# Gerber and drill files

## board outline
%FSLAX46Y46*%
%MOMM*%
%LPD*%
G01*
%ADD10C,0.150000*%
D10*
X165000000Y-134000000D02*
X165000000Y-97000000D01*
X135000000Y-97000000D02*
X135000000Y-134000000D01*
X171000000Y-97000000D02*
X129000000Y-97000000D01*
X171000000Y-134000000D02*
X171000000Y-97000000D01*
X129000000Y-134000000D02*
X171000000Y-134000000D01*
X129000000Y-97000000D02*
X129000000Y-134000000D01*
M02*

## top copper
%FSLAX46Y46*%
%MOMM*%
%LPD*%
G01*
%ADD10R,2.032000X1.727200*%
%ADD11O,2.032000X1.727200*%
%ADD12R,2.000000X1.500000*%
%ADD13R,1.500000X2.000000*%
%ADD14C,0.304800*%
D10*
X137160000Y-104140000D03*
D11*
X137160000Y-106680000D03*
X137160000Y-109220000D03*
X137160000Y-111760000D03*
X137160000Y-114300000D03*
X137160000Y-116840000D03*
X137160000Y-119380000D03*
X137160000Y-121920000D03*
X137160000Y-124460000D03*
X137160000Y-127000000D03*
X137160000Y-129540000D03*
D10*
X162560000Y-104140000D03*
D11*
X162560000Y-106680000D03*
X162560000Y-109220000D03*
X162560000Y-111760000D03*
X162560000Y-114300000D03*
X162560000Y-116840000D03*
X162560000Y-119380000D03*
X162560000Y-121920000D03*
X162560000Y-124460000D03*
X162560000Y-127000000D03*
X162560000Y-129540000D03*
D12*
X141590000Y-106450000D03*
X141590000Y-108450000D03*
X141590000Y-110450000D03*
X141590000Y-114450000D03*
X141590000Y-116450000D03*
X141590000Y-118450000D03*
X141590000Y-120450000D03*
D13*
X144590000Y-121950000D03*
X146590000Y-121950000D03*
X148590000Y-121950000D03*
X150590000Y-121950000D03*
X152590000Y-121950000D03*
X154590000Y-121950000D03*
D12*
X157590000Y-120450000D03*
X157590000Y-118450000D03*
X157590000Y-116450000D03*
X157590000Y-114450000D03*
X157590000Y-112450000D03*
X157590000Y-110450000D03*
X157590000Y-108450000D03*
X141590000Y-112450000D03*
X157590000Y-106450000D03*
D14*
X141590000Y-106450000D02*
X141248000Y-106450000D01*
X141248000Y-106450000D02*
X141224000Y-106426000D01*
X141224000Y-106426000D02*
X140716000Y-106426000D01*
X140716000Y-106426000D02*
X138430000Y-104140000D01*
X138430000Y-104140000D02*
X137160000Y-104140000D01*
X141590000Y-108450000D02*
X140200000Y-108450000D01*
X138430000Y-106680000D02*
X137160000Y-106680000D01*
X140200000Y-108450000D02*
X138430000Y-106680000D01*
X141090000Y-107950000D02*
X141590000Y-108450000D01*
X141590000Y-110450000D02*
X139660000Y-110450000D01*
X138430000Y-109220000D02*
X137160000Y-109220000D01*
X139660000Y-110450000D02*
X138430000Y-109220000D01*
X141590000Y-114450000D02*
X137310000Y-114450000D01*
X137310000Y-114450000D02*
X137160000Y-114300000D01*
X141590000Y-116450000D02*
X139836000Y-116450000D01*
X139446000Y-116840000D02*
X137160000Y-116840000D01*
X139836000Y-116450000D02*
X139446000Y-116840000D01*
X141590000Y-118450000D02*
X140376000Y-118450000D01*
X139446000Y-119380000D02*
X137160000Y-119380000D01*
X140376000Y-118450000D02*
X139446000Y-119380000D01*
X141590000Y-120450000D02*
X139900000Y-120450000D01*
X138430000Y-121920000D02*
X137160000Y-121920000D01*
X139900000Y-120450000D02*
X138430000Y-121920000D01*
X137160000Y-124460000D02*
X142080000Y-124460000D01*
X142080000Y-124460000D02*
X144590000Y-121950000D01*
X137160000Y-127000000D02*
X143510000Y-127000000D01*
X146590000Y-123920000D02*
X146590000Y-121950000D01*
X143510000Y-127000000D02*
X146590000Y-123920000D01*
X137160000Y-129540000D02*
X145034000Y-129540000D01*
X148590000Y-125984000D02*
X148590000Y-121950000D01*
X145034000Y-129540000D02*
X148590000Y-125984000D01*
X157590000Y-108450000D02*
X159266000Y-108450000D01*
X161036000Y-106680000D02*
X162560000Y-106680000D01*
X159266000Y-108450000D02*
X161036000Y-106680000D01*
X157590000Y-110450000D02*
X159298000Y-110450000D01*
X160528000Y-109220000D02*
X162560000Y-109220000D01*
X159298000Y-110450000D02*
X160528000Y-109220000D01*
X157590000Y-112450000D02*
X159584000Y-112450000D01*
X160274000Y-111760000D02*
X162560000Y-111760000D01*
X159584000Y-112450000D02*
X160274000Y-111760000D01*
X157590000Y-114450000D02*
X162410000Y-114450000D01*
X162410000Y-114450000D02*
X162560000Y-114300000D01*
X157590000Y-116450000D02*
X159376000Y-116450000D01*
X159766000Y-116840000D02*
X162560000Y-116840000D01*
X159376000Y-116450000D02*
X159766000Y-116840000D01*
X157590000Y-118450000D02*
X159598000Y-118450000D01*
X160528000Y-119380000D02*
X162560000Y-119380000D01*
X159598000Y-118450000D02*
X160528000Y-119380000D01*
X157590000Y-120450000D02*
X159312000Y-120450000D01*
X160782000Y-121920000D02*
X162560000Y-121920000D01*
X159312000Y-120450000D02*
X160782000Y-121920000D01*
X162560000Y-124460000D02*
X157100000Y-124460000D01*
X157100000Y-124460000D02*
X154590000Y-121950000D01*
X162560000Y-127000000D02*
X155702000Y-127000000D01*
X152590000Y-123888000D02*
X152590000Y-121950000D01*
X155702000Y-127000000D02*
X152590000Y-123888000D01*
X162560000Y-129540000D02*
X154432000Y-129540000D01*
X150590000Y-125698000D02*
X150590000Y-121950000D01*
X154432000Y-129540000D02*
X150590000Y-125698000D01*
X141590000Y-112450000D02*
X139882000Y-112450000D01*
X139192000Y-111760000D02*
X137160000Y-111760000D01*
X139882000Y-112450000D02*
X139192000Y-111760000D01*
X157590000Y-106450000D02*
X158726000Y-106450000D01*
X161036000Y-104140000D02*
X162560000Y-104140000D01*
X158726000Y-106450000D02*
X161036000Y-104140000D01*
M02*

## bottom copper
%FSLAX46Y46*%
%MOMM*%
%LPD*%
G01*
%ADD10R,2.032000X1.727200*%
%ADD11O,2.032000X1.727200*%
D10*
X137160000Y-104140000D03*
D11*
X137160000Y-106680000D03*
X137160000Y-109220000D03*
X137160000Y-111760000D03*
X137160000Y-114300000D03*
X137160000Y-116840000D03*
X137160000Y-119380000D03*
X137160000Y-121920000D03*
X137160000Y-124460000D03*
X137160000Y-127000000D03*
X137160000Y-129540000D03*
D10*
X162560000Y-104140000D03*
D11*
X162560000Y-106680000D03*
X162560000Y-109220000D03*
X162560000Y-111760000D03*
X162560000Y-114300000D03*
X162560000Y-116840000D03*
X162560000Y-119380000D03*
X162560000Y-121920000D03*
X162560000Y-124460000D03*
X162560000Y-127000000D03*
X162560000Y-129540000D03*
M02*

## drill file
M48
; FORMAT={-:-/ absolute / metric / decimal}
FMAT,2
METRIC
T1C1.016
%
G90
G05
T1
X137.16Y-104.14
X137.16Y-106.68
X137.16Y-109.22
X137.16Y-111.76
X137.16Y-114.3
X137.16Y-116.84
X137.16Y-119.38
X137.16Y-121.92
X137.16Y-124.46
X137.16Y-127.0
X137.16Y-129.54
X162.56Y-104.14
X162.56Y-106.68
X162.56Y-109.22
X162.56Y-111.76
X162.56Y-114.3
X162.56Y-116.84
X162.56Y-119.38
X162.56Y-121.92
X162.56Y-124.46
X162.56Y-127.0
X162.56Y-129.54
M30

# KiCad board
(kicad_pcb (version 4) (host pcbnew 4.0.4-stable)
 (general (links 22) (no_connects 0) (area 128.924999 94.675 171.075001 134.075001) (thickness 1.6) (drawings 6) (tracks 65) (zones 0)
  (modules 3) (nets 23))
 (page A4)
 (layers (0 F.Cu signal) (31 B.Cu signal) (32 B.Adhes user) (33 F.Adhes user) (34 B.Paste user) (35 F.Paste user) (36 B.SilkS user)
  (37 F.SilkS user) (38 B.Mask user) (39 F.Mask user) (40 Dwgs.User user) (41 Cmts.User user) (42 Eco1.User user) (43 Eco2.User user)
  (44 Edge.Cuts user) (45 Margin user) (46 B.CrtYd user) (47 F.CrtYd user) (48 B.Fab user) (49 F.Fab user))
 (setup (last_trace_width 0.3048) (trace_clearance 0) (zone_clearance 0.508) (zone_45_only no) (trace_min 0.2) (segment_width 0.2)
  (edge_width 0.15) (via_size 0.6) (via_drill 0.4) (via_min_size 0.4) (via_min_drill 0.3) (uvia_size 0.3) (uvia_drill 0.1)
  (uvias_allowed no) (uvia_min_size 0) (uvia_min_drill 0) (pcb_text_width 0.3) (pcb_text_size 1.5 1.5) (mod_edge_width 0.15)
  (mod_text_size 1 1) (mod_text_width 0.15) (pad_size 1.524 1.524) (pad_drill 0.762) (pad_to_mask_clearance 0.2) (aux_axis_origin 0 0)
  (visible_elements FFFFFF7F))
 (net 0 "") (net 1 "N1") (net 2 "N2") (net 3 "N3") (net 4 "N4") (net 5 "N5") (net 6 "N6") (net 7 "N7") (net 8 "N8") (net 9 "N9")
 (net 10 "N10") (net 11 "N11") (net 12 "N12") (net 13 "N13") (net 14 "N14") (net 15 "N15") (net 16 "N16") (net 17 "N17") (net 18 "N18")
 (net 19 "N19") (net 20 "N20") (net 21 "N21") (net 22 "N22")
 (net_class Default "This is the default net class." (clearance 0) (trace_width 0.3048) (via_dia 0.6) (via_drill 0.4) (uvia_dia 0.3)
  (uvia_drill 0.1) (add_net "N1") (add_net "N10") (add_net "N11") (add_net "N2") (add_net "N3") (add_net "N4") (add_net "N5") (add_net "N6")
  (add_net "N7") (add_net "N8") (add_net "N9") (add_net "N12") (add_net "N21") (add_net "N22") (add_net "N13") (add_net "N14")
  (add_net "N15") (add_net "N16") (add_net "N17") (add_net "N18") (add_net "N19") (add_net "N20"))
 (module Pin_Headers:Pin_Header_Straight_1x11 (layer F.Cu) (at 137.16 104.14)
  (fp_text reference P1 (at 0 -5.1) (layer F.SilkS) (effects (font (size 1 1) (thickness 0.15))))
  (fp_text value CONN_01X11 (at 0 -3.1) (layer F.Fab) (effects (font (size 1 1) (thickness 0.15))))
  (pad 1 thru_hole rect (at 0 0) (size 2.032 1.7272) (drill 1.016) (layers *.Cu *.Mask F.SilkS) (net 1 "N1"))
  (pad 2 thru_hole oval (at 0 2.54) (size 2.032 1.7272) (drill 1.016) (layers *.Cu *.Mask F.SilkS) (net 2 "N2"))
  (pad 3 thru_hole oval (at 0 5.08) (size 2.032 1.7272) (drill 1.016) (layers *.Cu *.Mask F.SilkS) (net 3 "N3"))
  (pad 4 thru_hole oval (at 0 7.62) (size 2.032 1.7272) (drill 1.016) (layers *.Cu *.Mask F.SilkS) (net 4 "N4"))
  (pad 5 thru_hole oval (at 0 10.16) (size 2.032 1.7272) (drill 1.016) (layers *.Cu *.Mask F.SilkS) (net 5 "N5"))
  (pad 6 thru_hole oval (at 0 12.7) (size 2.032 1.7272) (drill 1.016) (layers *.Cu *.Mask F.SilkS) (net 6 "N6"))
  (pad 7 thru_hole oval (at 0 15.24) (size 2.032 1.7272) (drill 1.016) (layers *.Cu *.Mask F.SilkS) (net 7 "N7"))
  (pad 8 thru_hole oval (at 0 17.78) (size 2.032 1.7272) (drill 1.016) (layers *.Cu *.Mask F.SilkS) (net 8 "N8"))
  (pad 9 thru_hole oval (at 0 20.32) (size 2.032 1.7272) (drill 1.016) (layers *.Cu *.Mask F.SilkS) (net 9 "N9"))
  (pad 10 thru_hole oval (at 0 22.86) (size 2.032 1.7272) (drill 1.016) (layers *.Cu *.Mask F.SilkS) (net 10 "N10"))
  (pad 11 thru_hole oval (at 0 25.4) (size 2.032 1.7272) (drill 1.016) (layers *.Cu *.Mask F.SilkS) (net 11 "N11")))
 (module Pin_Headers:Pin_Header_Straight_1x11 (layer F.Cu) (at 162.56 104.14)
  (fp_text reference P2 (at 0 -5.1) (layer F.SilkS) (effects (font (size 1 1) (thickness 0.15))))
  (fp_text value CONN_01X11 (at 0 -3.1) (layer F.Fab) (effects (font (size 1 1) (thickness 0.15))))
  (pad 1 thru_hole rect (at 0 0) (size 2.032 1.7272) (drill 1.016) (layers *.Cu *.Mask F.SilkS) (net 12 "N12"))
  (pad 2 thru_hole oval (at 0 2.54) (size 2.032 1.7272) (drill 1.016) (layers *.Cu *.Mask F.SilkS) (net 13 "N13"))
  (pad 3 thru_hole oval (at 0 5.08) (size 2.032 1.7272) (drill 1.016) (layers *.Cu *.Mask F.SilkS) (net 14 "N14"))
  (pad 4 thru_hole oval (at 0 7.62) (size 2.032 1.7272) (drill 1.016) (layers *.Cu *.Mask F.SilkS) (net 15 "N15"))
  (pad 5 thru_hole oval (at 0 10.16) (size 2.032 1.7272) (drill 1.016) (layers *.Cu *.Mask F.SilkS) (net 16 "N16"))
  (pad 6 thru_hole oval (at 0 12.7) (size 2.032 1.7272) (drill 1.016) (layers *.Cu *.Mask F.SilkS) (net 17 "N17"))
  (pad 7 thru_hole oval (at 0 15.24) (size 2.032 1.7272) (drill 1.016) (layers *.Cu *.Mask F.SilkS) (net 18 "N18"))
  (pad 8 thru_hole oval (at 0 17.78) (size 2.032 1.7272) (drill 1.016) (layers *.Cu *.Mask F.SilkS) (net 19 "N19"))
  (pad 9 thru_hole oval (at 0 20.32) (size 2.032 1.7272) (drill 1.016) (layers *.Cu *.Mask F.SilkS) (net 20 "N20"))
  (pad 10 thru_hole oval (at 0 22.86) (size 2.032 1.7272) (drill 1.016) (layers *.Cu *.Mask F.SilkS) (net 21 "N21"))
  (pad 11 thru_hole oval (at 0 25.4) (size 2.032 1.7272) (drill 1.016) (layers *.Cu *.Mask F.SilkS) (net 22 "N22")))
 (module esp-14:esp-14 (layer F.Cu) (at 148.59 107.95)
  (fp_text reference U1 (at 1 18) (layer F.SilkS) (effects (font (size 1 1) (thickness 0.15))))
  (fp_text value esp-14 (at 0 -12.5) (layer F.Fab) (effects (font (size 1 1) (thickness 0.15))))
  (pad 1 smd rect (at -7 -1.5) (size 2 1.5) (layers F.Cu F.Paste F.Mask) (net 1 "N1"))
  (pad 2 smd rect (at -7 0.5) (size 2 1.5) (layers F.Cu F.Paste F.Mask) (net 2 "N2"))
  (pad 3 smd rect (at -7 2.5) (size 2 1.5) (layers F.Cu F.Paste F.Mask) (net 3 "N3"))
  (pad 5 smd rect (at -7 6.5) (size 2 1.5) (layers F.Cu F.Paste F.Mask) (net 5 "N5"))
  (pad 6 smd rect (at -7 8.5) (size 2 1.5) (layers F.Cu F.Paste F.Mask) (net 6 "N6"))
  (pad 7 smd rect (at -7 10.5) (size 2 1.5) (layers F.Cu F.Paste F.Mask) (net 7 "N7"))
  (pad 8 smd rect (at -7 12.5) (size 2 1.5) (layers F.Cu F.Paste F.Mask) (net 8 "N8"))
  (pad 9 smd rect (at -4 14) (size 1.5 2) (layers F.Cu F.Paste F.Mask) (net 9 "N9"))
  (pad 10 smd rect (at -2 14) (size 1.5 2) (layers F.Cu F.Paste F.Mask) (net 10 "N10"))
  (pad 11 smd rect (at 0 14) (size 1.5 2) (layers F.Cu F.Paste F.Mask) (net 11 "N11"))
  (pad 12 smd rect (at 2 14) (size 1.5 2) (layers F.Cu F.Paste F.Mask) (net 22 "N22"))
  (pad 13 smd rect (at 4 14) (size 1.5 2) (layers F.Cu F.Paste F.Mask) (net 21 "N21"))
  (pad 14 smd rect (at 6 14) (size 1.5 2) (layers F.Cu F.Paste F.Mask) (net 20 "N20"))
  (pad 15 smd rect (at 9 12.5) (size 2 1.5) (layers F.Cu F.Paste F.Mask) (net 19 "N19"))
  (pad 16 smd rect (at 9 10.5) (size 2 1.5) (layers F.Cu F.Paste F.Mask) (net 18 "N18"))
  (pad 17 smd rect (at 9 8.5) (size 2 1.5) (layers F.Cu F.Paste F.Mask) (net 17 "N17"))
  (pad 18 smd rect (at 9 6.5) (size 2 1.5) (layers F.Cu F.Paste F.Mask) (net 16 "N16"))
  (pad 19 smd rect (at 9 4.5) (size 2 1.5) (layers F.Cu F.Paste F.Mask) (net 15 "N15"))
  (pad 20 smd rect (at 9 2.5) (size 2 1.5) (layers F.Cu F.Paste F.Mask) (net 14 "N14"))
  (pad 21 smd rect (at 9 0.5) (size 2 1.5) (layers F.Cu F.Paste F.Mask) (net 13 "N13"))
  (pad 4 smd rect (at -7 4.5) (size 2 1.5) (layers F.Cu F.Paste F.Mask) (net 4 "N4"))
  (pad 22 smd rect (at 9 -1.5) (size 2 1.5) (layers F.Cu F.Paste F.Mask) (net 12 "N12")))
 (gr_line (start 165 134) (end 165 97) (angle 90) (layer Edge.Cuts) (width 0.15))
 (gr_line (start 135 97) (end 135 134) (angle 90) (layer Edge.Cuts) (width 0.15))
 (gr_line (start 171 97) (end 129 97) (angle 90) (layer Edge.Cuts) (width 0.15))
 (gr_line (start 171 134) (end 171 97) (angle 90) (layer Edge.Cuts) (width 0.15))
 (gr_line (start 129 134) (end 171 134) (angle 90) (layer Edge.Cuts) (width 0.15))
 (gr_line (start 129 97) (end 129 134) (angle 90) (layer Edge.Cuts) (width 0.15))
 (segment (start 141.59 106.45) (end 141.248 106.45) (width 0.3048) (layer F.Cu) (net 1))
 (segment (start 141.248 106.45) (end 141.224 106.426) (width 0.3048) (layer F.Cu) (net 1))
 (segment (start 141.224 106.426) (end 140.716 106.426) (width 0.3048) (layer F.Cu) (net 1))
 (segment (start 140.716 106.426) (end 138.43 104.14) (width 0.3048) (layer F.Cu) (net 1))
 (segment (start 138.43 104.14) (end 137.16 104.14) (width 0.3048) (layer F.Cu) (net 1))
 (segment (start 141.59 108.45) (end 140.2 108.45) (width 0.3048) (layer F.Cu) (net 2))
 (segment (start 138.43 106.68) (end 137.16 106.68) (width 0.3048) (layer F.Cu) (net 2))
 (segment (start 140.2 108.45) (end 138.43 106.68) (width 0.3048) (layer F.Cu) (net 2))
 (segment (start 141.09 107.95) (end 141.59 108.45) (width 0.3048) (layer F.Cu) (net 2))
 (segment (start 141.59 110.45) (end 139.66 110.45) (width 0.3048) (layer F.Cu) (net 3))
 (segment (start 138.43 109.22) (end 137.16 109.22) (width 0.3048) (layer F.Cu) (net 3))
 (segment (start 139.66 110.45) (end 138.43 109.22) (width 0.3048) (layer F.Cu) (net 3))
 (segment (start 141.59 114.45) (end 137.31 114.45) (width 0.3048) (layer F.Cu) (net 5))
 (segment (start 137.31 114.45) (end 137.16 114.3) (width 0.3048) (layer F.Cu) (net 5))
 (segment (start 141.59 116.45) (end 139.836 116.45) (width 0.3048) (layer F.Cu) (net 6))
 (segment (start 139.446 116.84) (end 137.16 116.84) (width 0.3048) (layer F.Cu) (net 6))
 (segment (start 139.836 116.45) (end 139.446 116.84) (width 0.3048) (layer F.Cu) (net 6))
 (segment (start 141.59 118.45) (end 140.376 118.45) (width 0.3048) (layer F.Cu) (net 7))
 (segment (start 139.446 119.38) (end 137.16 119.38) (width 0.3048) (layer F.Cu) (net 7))
 (segment (start 140.376 118.45) (end 139.446 119.38) (width 0.3048) (layer F.Cu) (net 7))
 (segment (start 141.59 120.45) (end 139.9 120.45) (width 0.3048) (layer F.Cu) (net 8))
 (segment (start 138.43 121.92) (end 137.16 121.92) (width 0.3048) (layer F.Cu) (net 8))
 (segment (start 139.9 120.45) (end 138.43 121.92) (width 0.3048) (layer F.Cu) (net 8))
 (segment (start 137.16 124.46) (end 142.08 124.46) (width 0.3048) (layer F.Cu) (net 9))
 (segment (start 142.08 124.46) (end 144.59 121.95) (width 0.3048) (layer F.Cu) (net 9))
 (segment (start 137.16 127) (end 143.51 127) (width 0.3048) (layer F.Cu) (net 10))
 (segment (start 146.59 123.92) (end 146.59 121.95) (width 0.3048) (layer F.Cu) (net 10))
 (segment (start 143.51 127) (end 146.59 123.92) (width 0.3048) (layer F.Cu) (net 10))
 (segment (start 137.16 129.54) (end 145.034 129.54) (width 0.3048) (layer F.Cu) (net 11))
 (segment (start 148.59 125.984) (end 148.59 121.95) (width 0.3048) (layer F.Cu) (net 11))
 (segment (start 145.034 129.54) (end 148.59 125.984) (width 0.3048) (layer F.Cu) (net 11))
 (segment (start 157.59 108.45) (end 159.266 108.45) (width 0.3048) (layer F.Cu) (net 13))
 (segment (start 161.036 106.68) (end 162.56 106.68) (width 0.3048) (layer F.Cu) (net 13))
 (segment (start 159.266 108.45) (end 161.036 106.68) (width 0.3048) (layer F.Cu) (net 13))
 (segment (start 157.59 110.45) (end 159.298 110.45) (width 0.3048) (layer F.Cu) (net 14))
 (segment (start 160.528 109.22) (end 162.56 109.22) (width 0.3048) (layer F.Cu) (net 14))
 (segment (start 159.298 110.45) (end 160.528 109.22) (width 0.3048) (layer F.Cu) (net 14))
 (segment (start 157.59 112.45) (end 159.584 112.45) (width 0.3048) (layer F.Cu) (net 15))
 (segment (start 160.274 111.76) (end 162.56 111.76) (width 0.3048) (layer F.Cu) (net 15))
 (segment (start 159.584 112.45) (end 160.274 111.76) (width 0.3048) (layer F.Cu) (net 15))
 (segment (start 157.59 114.45) (end 162.41 114.45) (width 0.3048) (layer F.Cu) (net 16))
 (segment (start 162.41 114.45) (end 162.56 114.3) (width 0.3048) (layer F.Cu) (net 16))
 (segment (start 157.59 116.45) (end 159.376 116.45) (width 0.3048) (layer F.Cu) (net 17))
 (segment (start 159.766 116.84) (end 162.56 116.84) (width 0.3048) (layer F.Cu) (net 17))
 (segment (start 159.376 116.45) (end 159.766 116.84) (width 0.3048) (layer F.Cu) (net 17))
 (segment (start 157.59 118.45) (end 159.598 118.45) (width 0.3048) (layer F.Cu) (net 18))
 (segment (start 160.528 119.38) (end 162.56 119.38) (width 0.3048) (layer F.Cu) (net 18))
 (segment (start 159.598 118.45) (end 160.528 119.38) (width 0.3048) (layer F.Cu) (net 18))
 (segment (start 157.59 120.45) (end 159.312 120.45) (width 0.3048) (layer F.Cu) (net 19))
 (segment (start 160.782 121.92) (end 162.56 121.92) (width 0.3048) (layer F.Cu) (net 19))
 (segment (start 159.312 120.45) (end 160.782 121.92) (width 0.3048) (layer F.Cu) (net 19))
 (segment (start 162.56 124.46) (end 157.1 124.46) (width 0.3048) (layer F.Cu) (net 20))
 (segment (start 157.1 124.46) (end 154.59 121.95) (width 0.3048) (layer F.Cu) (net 20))
 (segment (start 162.56 127) (end 155.702 127) (width 0.3048) (layer F.Cu) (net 21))
 (segment (start 152.59 123.888) (end 152.59 121.95) (width 0.3048) (layer F.Cu) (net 21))
 (segment (start 155.702 127) (end 152.59 123.888) (width 0.3048) (layer F.Cu) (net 21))
 (segment (start 162.56 129.54) (end 154.432 129.54) (width 0.3048) (layer F.Cu) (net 22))
 (segment (start 150.59 125.698) (end 150.59 121.95) (width 0.3048) (layer F.Cu) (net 22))
 (segment (start 154.432 129.54) (end 150.59 125.698) (width 0.3048) (layer F.Cu) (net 22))
 (segment (start 141.59 112.45) (end 139.882 112.45) (width 0.3048) (layer F.Cu) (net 4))
 (segment (start 139.192 111.76) (end 137.16 111.76) (width 0.3048) (layer F.Cu) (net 4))
 (segment (start 139.882 112.45) (end 139.192 111.76) (width 0.3048) (layer F.Cu) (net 4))
 (segment (start 157.59 106.45) (end 158.726 106.45) (width 0.3048) (layer F.Cu) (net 12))
 (segment (start 161.036 104.14) (end 162.56 104.14) (width 0.3048) (layer F.Cu) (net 12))
 (segment (start 158.726 106.45) (end 161.036 104.14) (width 0.3048) (layer F.Cu) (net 12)))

